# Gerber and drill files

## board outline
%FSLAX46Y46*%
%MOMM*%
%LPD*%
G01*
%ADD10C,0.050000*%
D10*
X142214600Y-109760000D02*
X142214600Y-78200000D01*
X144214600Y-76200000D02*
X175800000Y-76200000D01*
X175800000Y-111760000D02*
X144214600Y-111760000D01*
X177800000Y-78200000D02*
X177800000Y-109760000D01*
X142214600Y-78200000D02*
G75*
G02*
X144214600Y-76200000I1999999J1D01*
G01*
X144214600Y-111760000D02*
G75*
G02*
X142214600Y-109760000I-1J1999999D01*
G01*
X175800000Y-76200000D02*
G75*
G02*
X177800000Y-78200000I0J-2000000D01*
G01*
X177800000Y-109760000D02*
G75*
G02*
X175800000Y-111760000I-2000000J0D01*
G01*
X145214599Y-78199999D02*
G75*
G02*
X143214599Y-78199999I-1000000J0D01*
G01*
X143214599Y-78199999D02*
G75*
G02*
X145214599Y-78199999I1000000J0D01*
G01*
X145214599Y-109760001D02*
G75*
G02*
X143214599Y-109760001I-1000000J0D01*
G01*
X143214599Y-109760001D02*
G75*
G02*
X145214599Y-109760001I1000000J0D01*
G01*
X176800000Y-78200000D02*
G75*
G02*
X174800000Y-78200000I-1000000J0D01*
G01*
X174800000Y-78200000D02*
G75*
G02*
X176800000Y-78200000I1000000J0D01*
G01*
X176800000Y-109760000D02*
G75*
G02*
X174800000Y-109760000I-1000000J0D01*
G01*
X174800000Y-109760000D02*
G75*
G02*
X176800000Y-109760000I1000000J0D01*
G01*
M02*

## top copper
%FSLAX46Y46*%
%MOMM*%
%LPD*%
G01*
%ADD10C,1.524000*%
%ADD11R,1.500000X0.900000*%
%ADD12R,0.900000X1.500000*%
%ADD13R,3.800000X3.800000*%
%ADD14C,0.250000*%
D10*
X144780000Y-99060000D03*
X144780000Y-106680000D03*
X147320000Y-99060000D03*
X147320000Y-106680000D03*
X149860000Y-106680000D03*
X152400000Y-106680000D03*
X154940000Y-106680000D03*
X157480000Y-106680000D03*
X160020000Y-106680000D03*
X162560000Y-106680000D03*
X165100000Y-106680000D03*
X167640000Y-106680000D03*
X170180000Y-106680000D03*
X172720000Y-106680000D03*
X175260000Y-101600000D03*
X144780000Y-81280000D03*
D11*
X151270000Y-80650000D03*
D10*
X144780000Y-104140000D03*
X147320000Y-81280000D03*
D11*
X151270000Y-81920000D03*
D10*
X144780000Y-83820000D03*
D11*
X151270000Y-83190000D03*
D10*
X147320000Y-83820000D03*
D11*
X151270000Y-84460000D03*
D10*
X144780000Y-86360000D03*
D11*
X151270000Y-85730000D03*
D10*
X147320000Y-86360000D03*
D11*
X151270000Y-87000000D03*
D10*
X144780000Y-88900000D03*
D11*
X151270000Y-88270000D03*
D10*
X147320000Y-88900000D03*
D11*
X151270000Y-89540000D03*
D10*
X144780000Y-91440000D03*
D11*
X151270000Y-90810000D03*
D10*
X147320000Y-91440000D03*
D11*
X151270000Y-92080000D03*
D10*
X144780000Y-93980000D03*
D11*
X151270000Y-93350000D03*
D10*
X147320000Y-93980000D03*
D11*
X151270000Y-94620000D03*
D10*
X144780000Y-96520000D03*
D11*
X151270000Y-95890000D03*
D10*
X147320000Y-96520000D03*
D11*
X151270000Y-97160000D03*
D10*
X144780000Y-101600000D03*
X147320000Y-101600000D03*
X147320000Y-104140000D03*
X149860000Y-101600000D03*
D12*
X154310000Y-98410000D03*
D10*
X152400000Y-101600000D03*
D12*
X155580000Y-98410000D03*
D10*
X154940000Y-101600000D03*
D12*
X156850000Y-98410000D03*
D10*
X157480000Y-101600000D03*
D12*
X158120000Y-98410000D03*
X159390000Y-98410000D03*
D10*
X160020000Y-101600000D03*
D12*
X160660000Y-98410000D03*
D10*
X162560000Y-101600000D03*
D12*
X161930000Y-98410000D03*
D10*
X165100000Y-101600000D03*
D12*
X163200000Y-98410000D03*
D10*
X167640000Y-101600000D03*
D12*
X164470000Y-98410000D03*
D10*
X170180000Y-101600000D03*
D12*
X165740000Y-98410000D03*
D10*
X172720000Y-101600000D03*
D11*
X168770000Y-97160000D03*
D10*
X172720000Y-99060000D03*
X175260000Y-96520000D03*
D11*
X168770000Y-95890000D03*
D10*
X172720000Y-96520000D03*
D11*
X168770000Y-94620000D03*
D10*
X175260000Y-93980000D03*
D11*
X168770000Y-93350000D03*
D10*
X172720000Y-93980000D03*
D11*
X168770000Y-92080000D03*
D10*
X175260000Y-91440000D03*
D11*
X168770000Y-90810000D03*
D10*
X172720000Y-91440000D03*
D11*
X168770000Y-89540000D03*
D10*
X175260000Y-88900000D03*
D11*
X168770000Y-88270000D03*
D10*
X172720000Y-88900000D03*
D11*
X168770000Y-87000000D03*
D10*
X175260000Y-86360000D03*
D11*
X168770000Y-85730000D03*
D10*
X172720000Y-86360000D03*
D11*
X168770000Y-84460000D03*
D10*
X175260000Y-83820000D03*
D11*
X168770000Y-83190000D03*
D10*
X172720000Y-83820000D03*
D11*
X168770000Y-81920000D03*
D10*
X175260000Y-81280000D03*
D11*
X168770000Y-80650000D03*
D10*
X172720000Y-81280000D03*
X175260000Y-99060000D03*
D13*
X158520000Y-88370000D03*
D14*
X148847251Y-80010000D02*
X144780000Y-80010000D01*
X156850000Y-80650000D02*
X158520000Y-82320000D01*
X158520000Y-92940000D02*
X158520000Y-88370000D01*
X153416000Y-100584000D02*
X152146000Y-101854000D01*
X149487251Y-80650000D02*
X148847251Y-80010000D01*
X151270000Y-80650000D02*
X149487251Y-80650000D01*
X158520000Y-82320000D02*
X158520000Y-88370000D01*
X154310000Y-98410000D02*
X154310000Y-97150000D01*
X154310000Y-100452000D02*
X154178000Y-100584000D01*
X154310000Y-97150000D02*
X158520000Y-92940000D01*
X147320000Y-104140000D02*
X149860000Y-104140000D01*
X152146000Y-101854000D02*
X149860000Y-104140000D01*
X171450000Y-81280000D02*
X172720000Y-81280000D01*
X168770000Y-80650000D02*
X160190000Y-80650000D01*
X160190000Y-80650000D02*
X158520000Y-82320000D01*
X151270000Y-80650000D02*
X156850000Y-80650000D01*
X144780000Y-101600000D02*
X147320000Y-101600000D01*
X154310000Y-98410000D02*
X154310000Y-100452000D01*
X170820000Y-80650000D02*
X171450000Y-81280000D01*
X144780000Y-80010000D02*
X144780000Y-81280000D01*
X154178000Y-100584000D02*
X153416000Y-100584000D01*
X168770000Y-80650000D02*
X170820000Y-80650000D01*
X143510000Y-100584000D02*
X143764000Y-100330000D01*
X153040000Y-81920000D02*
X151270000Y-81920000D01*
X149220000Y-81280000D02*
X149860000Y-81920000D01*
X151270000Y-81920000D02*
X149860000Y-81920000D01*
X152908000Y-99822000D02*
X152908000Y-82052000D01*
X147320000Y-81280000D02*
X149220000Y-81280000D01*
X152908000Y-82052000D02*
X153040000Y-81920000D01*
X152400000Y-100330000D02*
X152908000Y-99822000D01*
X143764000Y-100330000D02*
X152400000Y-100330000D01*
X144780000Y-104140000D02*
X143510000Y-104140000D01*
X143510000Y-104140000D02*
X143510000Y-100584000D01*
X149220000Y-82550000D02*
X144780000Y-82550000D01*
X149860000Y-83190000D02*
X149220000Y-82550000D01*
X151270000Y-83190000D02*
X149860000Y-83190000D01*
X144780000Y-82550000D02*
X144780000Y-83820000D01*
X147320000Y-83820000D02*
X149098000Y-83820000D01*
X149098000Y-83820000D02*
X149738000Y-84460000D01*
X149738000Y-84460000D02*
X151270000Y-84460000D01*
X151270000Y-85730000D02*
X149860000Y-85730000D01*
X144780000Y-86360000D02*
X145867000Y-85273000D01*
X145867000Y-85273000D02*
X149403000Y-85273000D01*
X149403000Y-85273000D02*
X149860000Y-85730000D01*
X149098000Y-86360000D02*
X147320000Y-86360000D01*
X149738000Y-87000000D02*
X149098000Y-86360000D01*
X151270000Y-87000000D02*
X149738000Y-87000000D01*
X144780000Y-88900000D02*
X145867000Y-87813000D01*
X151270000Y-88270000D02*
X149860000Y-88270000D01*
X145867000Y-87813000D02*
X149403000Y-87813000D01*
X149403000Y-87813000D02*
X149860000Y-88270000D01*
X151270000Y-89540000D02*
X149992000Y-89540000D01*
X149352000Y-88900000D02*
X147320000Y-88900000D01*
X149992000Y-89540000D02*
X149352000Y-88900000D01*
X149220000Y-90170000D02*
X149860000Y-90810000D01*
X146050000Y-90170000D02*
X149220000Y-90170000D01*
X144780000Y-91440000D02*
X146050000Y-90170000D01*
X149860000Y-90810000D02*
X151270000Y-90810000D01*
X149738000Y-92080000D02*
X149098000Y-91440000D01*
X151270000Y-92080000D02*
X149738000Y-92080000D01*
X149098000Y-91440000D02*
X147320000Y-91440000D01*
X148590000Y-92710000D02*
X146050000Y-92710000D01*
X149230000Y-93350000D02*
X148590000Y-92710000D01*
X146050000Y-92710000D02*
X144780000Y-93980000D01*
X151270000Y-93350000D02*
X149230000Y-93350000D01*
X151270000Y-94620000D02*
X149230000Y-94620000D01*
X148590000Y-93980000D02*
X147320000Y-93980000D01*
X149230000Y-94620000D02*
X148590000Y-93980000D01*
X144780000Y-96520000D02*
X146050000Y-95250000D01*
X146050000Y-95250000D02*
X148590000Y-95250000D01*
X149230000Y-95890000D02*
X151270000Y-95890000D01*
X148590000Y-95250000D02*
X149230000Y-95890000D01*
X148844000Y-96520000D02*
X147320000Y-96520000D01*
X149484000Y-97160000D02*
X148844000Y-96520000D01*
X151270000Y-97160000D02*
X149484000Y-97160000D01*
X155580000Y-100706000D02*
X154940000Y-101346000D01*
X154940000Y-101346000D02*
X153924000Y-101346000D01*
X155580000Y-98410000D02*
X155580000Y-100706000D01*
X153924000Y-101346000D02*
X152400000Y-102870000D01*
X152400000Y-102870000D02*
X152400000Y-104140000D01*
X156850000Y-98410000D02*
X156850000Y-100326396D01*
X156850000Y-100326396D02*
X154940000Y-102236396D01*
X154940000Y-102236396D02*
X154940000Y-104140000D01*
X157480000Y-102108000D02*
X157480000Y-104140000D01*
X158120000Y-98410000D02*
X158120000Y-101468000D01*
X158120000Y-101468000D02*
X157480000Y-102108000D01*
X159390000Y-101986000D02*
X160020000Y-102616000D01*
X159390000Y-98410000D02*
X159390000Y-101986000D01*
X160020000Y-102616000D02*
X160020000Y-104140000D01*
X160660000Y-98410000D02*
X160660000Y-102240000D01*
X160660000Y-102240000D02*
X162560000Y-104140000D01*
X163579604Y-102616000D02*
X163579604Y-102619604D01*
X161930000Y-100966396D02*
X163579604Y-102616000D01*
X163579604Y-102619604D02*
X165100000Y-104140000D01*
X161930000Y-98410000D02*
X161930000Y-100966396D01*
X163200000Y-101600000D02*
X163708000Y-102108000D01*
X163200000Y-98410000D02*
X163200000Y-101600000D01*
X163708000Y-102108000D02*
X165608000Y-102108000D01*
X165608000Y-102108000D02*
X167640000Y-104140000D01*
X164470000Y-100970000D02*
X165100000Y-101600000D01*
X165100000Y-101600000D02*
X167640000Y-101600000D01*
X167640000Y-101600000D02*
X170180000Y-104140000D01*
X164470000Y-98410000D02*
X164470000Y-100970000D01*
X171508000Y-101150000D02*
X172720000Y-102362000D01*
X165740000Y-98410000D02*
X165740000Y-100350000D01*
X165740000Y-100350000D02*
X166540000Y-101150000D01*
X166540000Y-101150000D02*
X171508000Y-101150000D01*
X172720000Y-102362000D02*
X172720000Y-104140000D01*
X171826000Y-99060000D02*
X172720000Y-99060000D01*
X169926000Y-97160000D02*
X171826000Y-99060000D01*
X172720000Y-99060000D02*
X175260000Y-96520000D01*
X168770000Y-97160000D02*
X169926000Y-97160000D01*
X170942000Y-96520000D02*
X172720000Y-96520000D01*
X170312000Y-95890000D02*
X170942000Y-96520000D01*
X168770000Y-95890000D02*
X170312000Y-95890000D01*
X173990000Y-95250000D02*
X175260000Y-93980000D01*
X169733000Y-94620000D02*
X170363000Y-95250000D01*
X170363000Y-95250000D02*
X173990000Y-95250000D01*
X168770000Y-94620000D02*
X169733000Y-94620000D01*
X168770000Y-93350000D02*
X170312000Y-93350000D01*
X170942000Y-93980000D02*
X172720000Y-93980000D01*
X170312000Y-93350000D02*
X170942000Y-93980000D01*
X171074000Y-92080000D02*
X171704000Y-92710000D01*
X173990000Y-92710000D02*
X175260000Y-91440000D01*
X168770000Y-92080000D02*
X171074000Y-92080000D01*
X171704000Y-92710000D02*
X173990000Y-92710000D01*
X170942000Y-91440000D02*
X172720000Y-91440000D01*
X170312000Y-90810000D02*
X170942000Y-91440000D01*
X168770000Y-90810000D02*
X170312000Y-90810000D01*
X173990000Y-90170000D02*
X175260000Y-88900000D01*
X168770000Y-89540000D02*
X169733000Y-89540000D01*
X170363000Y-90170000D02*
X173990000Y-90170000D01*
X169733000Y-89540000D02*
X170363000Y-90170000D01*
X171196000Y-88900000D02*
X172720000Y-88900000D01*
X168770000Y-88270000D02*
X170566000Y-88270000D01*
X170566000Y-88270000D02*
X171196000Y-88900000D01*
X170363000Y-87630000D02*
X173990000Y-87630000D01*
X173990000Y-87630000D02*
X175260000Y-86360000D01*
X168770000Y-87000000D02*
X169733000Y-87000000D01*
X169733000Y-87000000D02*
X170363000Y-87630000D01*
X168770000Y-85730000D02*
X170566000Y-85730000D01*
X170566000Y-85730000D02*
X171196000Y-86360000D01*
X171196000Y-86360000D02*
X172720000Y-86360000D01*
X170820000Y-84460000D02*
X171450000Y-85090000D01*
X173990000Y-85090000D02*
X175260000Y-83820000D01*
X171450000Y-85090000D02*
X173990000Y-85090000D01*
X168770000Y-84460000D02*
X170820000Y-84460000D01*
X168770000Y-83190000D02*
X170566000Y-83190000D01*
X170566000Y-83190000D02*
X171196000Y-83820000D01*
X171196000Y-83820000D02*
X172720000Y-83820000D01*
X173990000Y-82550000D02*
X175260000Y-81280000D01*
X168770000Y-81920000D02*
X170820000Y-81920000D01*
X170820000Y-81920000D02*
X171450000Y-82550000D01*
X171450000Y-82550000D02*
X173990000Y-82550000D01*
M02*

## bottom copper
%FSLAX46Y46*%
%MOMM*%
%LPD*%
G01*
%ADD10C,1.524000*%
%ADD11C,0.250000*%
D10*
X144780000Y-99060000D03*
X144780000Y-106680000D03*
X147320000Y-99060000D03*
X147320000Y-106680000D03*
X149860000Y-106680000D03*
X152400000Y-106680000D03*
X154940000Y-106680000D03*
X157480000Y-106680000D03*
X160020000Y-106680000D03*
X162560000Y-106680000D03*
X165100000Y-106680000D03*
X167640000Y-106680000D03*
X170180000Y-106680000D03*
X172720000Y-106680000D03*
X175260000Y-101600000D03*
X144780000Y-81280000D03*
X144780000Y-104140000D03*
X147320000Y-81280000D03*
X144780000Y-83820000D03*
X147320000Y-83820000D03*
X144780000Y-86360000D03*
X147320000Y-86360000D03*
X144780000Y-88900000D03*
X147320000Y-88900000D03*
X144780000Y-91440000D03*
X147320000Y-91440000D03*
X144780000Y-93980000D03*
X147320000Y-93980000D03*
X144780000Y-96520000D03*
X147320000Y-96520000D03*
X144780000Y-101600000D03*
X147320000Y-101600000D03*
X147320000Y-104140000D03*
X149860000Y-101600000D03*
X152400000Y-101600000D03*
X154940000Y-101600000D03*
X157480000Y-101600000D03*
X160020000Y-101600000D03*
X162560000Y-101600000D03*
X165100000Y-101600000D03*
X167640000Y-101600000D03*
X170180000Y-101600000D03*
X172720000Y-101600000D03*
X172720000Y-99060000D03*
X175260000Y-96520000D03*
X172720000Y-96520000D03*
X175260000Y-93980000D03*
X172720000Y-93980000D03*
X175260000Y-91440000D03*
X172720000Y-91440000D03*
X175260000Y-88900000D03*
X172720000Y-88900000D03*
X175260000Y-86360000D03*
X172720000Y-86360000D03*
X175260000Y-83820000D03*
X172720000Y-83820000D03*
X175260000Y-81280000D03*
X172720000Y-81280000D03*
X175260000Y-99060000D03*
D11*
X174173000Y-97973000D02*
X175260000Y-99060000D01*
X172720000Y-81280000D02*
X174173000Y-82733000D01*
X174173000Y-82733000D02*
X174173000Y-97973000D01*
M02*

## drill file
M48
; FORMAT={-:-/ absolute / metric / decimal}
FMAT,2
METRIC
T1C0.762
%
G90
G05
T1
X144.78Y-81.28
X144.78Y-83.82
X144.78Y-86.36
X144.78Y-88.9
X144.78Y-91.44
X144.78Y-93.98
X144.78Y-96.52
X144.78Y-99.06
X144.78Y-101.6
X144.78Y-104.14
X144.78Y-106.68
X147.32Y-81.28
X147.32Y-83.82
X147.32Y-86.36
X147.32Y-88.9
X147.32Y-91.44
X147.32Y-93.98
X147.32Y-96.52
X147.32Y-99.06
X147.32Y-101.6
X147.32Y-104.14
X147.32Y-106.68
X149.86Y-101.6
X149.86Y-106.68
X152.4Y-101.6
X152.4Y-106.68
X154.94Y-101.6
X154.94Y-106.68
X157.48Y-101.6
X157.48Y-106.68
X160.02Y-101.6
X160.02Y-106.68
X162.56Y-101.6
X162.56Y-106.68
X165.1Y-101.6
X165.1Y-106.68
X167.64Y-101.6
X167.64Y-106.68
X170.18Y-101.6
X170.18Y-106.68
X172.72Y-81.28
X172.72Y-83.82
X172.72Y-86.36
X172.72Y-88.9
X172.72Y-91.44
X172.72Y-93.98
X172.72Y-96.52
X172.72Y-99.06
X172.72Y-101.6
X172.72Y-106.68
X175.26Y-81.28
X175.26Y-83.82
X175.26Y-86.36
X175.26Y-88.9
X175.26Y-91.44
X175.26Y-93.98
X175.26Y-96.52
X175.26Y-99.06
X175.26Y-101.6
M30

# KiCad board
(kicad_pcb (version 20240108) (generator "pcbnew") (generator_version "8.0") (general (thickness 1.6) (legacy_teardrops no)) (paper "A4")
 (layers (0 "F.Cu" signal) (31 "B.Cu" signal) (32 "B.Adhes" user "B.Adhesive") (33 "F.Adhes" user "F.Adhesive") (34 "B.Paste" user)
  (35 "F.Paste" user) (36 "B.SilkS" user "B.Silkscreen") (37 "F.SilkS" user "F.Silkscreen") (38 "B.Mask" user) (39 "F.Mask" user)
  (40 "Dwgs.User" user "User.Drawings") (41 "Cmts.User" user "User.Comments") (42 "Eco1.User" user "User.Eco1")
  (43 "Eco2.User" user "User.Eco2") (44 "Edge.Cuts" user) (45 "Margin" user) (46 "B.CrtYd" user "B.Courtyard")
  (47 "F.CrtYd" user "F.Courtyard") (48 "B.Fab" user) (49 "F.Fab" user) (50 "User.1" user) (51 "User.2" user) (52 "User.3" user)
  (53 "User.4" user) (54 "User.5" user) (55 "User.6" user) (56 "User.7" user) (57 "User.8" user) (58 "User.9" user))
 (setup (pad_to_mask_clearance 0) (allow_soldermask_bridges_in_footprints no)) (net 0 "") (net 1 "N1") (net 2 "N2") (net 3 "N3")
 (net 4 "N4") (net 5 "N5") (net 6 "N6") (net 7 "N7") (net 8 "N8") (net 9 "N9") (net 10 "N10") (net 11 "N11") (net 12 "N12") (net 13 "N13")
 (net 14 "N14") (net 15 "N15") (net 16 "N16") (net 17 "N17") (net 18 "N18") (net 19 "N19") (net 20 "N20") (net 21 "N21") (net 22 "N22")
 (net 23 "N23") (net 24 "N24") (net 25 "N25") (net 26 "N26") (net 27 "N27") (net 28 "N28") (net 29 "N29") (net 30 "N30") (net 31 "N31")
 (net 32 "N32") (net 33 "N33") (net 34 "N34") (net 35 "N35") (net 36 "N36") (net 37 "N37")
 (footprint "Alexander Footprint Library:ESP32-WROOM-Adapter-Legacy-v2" (layer "F.Cu") (at 160.02 88.9)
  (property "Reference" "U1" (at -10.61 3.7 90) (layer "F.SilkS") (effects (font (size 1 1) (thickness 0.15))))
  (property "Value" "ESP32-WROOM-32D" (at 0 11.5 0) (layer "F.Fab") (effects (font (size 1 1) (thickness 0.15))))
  (fp_line (start -17.8054 20.86) (end -17.8054 -10.7) (stroke (width 0.05) (type default)) (layer "Edge.Cuts"))
  (fp_line (start -15.8054 -12.7) (end 15.78 -12.7) (stroke (width 0.05) (type default)) (layer "Edge.Cuts"))
  (fp_line (start 15.78 22.86) (end -15.8054 22.86) (stroke (width 0.05) (type default)) (layer "Edge.Cuts"))
  (fp_line (start 17.78 -10.7) (end 17.78 20.86) (stroke (width 0.05) (type default)) (layer "Edge.Cuts"))
  (fp_arc (start -17.8054 -10.7) (mid -17.219614 -12.114214) (end -15.8054 -12.7) (stroke (width 0.05) (type default)) (layer "Edge.Cuts"))
  (fp_arc (start -15.8054 22.86) (mid -17.219614 22.274214) (end -17.8054 20.86) (stroke (width 0.05) (type default)) (layer "Edge.Cuts"))
  (fp_arc (start 15.78 -12.7) (mid 17.194214 -12.114214) (end 17.78 -10.7) (stroke (width 0.05) (type default)) (layer "Edge.Cuts"))
  (fp_arc (start 17.78 20.86) (mid 17.194214 22.274214) (end 15.78 22.86) (stroke (width 0.05) (type default)) (layer "Edge.Cuts"))
  (fp_circle (center -15.805401 -10.700001) (end -14.805401 -10.700001) (stroke (width 0.05) (type default)) (fill none) (layer "Edge.Cuts"))
  (fp_circle (center -15.805401 20.860001) (end -14.805401 20.860001) (stroke (width 0.05) (type default)) (fill none) (layer "Edge.Cuts"))
  (fp_circle (center 15.78 -10.7) (end 16.78 -10.7) (stroke (width 0.05) (type default)) (fill none) (layer "Edge.Cuts"))
  (fp_circle (center 15.78 20.86) (end 16.78 20.86) (stroke (width 0.05) (type default)) (fill none) (layer "Edge.Cuts"))
  (pad "" thru_hole circle (at -15.24 10.16) (size 1.524 1.524) (drill 0.762) (layers "*.Cu" "*.Mask") (remove_unused_layers no))
  (pad "" thru_hole circle (at -15.24 17.78 90) (size 1.524 1.524) (drill 0.762) (layers "*.Cu" "*.Mask") (remove_unused_layers no))
  (pad "" thru_hole circle (at -12.7 10.16) (size 1.524 1.524) (drill 0.762) (layers "*.Cu" "*.Mask") (remove_unused_layers no))
  (pad "" thru_hole circle (at -12.7 17.78 90) (size 1.524 1.524) (drill 0.762) (layers "*.Cu" "*.Mask") (remove_unused_layers no))
  (pad "" thru_hole circle (at -10.16 17.78 90) (size 1.524 1.524) (drill 0.762) (layers "*.Cu" "*.Mask") (remove_unused_layers no))
  (pad "" thru_hole circle (at -7.62 17.78 90) (size 1.524 1.524) (drill 0.762) (layers "*.Cu" "*.Mask") (remove_unused_layers no))
  (pad "" thru_hole circle (at -5.08 17.78 90) (size 1.524 1.524) (drill 0.762) (layers "*.Cu" "*.Mask") (remove_unused_layers no))
  (pad "" thru_hole circle (at -2.54 17.78 90) (size 1.524 1.524) (drill 0.762) (layers "*.Cu" "*.Mask") (remove_unused_layers no))
  (pad "" thru_hole circle (at 0 17.78 90) (size 1.524 1.524) (drill 0.762) (layers "*.Cu" "*.Mask") (remove_unused_layers no))
  (pad "" thru_hole circle (at 2.54 17.78 90) (size 1.524 1.524) (drill 0.762) (layers "*.Cu" "*.Mask") (remove_unused_layers no))
  (pad "" thru_hole circle (at 5.08 17.78 90) (size 1.524 1.524) (drill 0.762) (layers "*.Cu" "*.Mask") (remove_unused_layers no))
  (pad "" thru_hole circle (at 7.62 17.78 90) (size 1.524 1.524) (drill 0.762) (layers "*.Cu" "*.Mask") (remove_unused_layers no))
  (pad "" thru_hole circle (at 10.16 17.78 90) (size 1.524 1.524) (drill 0.762) (layers "*.Cu" "*.Mask") (remove_unused_layers no))
  (pad "" thru_hole circle (at 12.7 17.78 90) (size 1.524 1.524) (drill 0.762) (layers "*.Cu" "*.Mask") (remove_unused_layers no))
  (pad "" thru_hole circle (at 15.24 12.7 90) (size 1.524 1.524) (drill 0.762) (layers "*.Cu" "*.Mask") (remove_unused_layers no))
  (pad "1" thru_hole circle (at -15.24 -7.62) (size 1.524 1.524) (drill 0.762) (layers "*.Cu" "*.Mask") (remove_unused_layers no)
   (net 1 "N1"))
  (pad "1" smd rect (at -8.75 -8.25) (size 1.5 0.9) (layers "F.Cu" "F.Paste" "F.Mask") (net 1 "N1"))
  (pad "2" thru_hole circle (at -15.24 15.24 90) (size 1.524 1.524) (drill 0.762) (layers "*.Cu" "*.Mask") (remove_unused_layers no)
   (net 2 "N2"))
  (pad "2" thru_hole circle (at -12.7 -7.62) (size 1.524 1.524) (drill 0.762) (layers "*.Cu" "*.Mask") (remove_unused_layers no)
   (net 2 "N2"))
  (pad "2" smd rect (at -8.75 -6.98) (size 1.5 0.9) (layers "F.Cu" "F.Paste" "F.Mask") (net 2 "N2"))
  (pad "3" thru_hole circle (at -15.24 -5.08) (size 1.524 1.524) (drill 0.762) (layers "*.Cu" "*.Mask") (remove_unused_layers no)
   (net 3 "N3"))
  (pad "3" smd rect (at -8.75 -5.71) (size 1.5 0.9) (layers "F.Cu" "F.Paste" "F.Mask") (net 3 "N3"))
  (pad "4" thru_hole circle (at -12.7 -5.08) (size 1.524 1.524) (drill 0.762) (layers "*.Cu" "*.Mask") (remove_unused_layers no)
   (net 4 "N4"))
  (pad "4" smd rect (at -8.75 -4.44) (size 1.5 0.9) (layers "F.Cu" "F.Paste" "F.Mask") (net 4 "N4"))
  (pad "5" thru_hole circle (at -15.24 -2.54) (size 1.524 1.524) (drill 0.762) (layers "*.Cu" "*.Mask") (remove_unused_layers no)
   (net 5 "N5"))
  (pad "5" smd rect (at -8.75 -3.17) (size 1.5 0.9) (layers "F.Cu" "F.Paste" "F.Mask") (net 5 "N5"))
  (pad "6" thru_hole circle (at -12.7 -2.54) (size 1.524 1.524) (drill 0.762) (layers "*.Cu" "*.Mask") (remove_unused_layers no)
   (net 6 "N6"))
  (pad "6" smd rect (at -8.75 -1.9) (size 1.5 0.9) (layers "F.Cu" "F.Paste" "F.Mask") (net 6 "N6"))
  (pad "7" thru_hole circle (at -15.24 0) (size 1.524 1.524) (drill 0.762) (layers "*.Cu" "*.Mask") (remove_unused_layers no) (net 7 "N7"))
  (pad "7" smd rect (at -8.75 -0.63) (size 1.5 0.9) (layers "F.Cu" "F.Paste" "F.Mask") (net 7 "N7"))
  (pad "8" thru_hole circle (at -12.7 0) (size 1.524 1.524) (drill 0.762) (layers "*.Cu" "*.Mask") (remove_unused_layers no) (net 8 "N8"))
  (pad "8" smd rect (at -8.75 0.64) (size 1.5 0.9) (layers "F.Cu" "F.Paste" "F.Mask") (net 8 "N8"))
  (pad "9" thru_hole circle (at -15.24 2.54) (size 1.524 1.524) (drill 0.762) (layers "*.Cu" "*.Mask") (remove_unused_layers no)
   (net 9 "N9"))
  (pad "9" smd rect (at -8.75 1.91) (size 1.5 0.9) (layers "F.Cu" "F.Paste" "F.Mask") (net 9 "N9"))
  (pad "10" thru_hole circle (at -12.7 2.54) (size 1.524 1.524) (drill 0.762) (layers "*.Cu" "*.Mask") (remove_unused_layers no)
   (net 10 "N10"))
  (pad "10" smd rect (at -8.75 3.18) (size 1.5 0.9) (layers "F.Cu" "F.Paste" "F.Mask") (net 10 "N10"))
  (pad "11" thru_hole circle (at -15.24 5.08) (size 1.524 1.524) (drill 0.762) (layers "*.Cu" "*.Mask") (remove_unused_layers no)
   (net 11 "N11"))
  (pad "11" smd rect (at -8.75 4.45) (size 1.5 0.9) (layers "F.Cu" "F.Paste" "F.Mask") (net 11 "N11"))
  (pad "12" thru_hole circle (at -12.7 5.08) (size 1.524 1.524) (drill 0.762) (layers "*.Cu" "*.Mask") (remove_unused_layers no)
   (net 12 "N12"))
  (pad "12" smd rect (at -8.75 5.72) (size 1.5 0.9) (layers "F.Cu" "F.Paste" "F.Mask") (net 12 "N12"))
  (pad "13" thru_hole circle (at -15.24 7.62) (size 1.524 1.524) (drill 0.762) (layers "*.Cu" "*.Mask") (remove_unused_layers no)
   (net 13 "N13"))
  (pad "13" smd rect (at -8.75 6.99) (size 1.5 0.9) (layers "F.Cu" "F.Paste" "F.Mask") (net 13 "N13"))
  (pad "14" thru_hole circle (at -12.7 7.62) (size 1.524 1.524) (drill 0.762) (layers "*.Cu" "*.Mask") (remove_unused_layers no)
   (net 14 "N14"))
  (pad "14" smd rect (at -8.75 8.26) (size 1.5 0.9) (layers "F.Cu" "F.Paste" "F.Mask") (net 14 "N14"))
  (pad "15" thru_hole circle (at -15.24 12.7 90) (size 1.524 1.524) (drill 0.762) (layers "*.Cu" "*.Mask") (remove_unused_layers no)
   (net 1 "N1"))
  (pad "15" thru_hole circle (at -12.7 12.7 90) (size 1.524 1.524) (drill 0.762) (layers "*.Cu" "*.Mask") (remove_unused_layers no)
   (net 1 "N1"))
  (pad "15" thru_hole circle (at -12.7 15.24 90) (size 1.524 1.524) (drill 0.762) (layers "*.Cu" "*.Mask") (remove_unused_layers no)
   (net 1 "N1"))
  (pad "15" thru_hole circle (at -10.16 12.7 90) (size 1.524 1.524) (drill 0.762) (layers "*.Cu" "*.Mask") (remove_unused_layers no)
   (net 1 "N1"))
  (pad "15" smd rect (at -5.71 9.51 90) (size 1.5 0.9) (layers "F.Cu" "F.Paste" "F.Mask") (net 1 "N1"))
  (pad "16" thru_hole circle (at -7.62 12.7 90) (size 1.524 1.524) (drill 0.762) (layers "*.Cu" "*.Mask") (remove_unused_layers no)
   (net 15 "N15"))
  (pad "16" smd rect (at -4.44 9.51 90) (size 1.5 0.9) (layers "F.Cu" "F.Paste" "F.Mask") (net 15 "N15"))
  (pad "17" thru_hole circle (at -5.08 12.7 90) (size 1.524 1.524) (drill 0.762) (layers "*.Cu" "*.Mask") (remove_unused_layers no)
   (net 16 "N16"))
  (pad "17" smd rect (at -3.17 9.51 90) (size 1.5 0.9) (layers "F.Cu" "F.Paste" "F.Mask") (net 16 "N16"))
  (pad "18" thru_hole circle (at -2.54 12.7 90) (size 1.524 1.524) (drill 0.762) (layers "*.Cu" "*.Mask") (remove_unused_layers no)
   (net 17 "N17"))
  (pad "18" smd rect (at -1.9 9.51 90) (size 1.5 0.9) (layers "F.Cu" "F.Paste" "F.Mask") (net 17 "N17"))
  (pad "19" smd rect (at -0.63 9.51 90) (size 1.5 0.9) (layers "F.Cu" "F.Paste" "F.Mask") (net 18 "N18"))
  (pad "19" thru_hole circle (at 0 12.7 90) (size 1.524 1.524) (drill 0.762) (layers "*.Cu" "*.Mask") (remove_unused_layers no)
   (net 18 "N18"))
  (pad "20" smd rect (at 0.64 9.51 90) (size 1.5 0.9) (layers "F.Cu" "F.Paste" "F.Mask") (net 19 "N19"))
  (pad "20" thru_hole circle (at 2.54 12.7 90) (size 1.524 1.524) (drill 0.762) (layers "*.Cu" "*.Mask") (remove_unused_layers no)
   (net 19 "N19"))
  (pad "21" smd rect (at 1.91 9.51 90) (size 1.5 0.9) (layers "F.Cu" "F.Paste" "F.Mask") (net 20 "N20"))
  (pad "21" thru_hole circle (at 5.08 12.7 90) (size 1.524 1.524) (drill 0.762) (layers "*.Cu" "*.Mask") (remove_unused_layers no)
   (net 20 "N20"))
  (pad "22" smd rect (at 3.18 9.51 90) (size 1.5 0.9) (layers "F.Cu" "F.Paste" "F.Mask") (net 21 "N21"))
  (pad "22" thru_hole circle (at 7.62 12.7 90) (size 1.524 1.524) (drill 0.762) (layers "*.Cu" "*.Mask") (remove_unused_layers no)
   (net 21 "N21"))
  (pad "23" smd rect (at 4.45 9.51 90) (size 1.5 0.9) (layers "F.Cu" "F.Paste" "F.Mask") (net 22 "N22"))
  (pad "23" thru_hole circle (at 10.16 12.7 90) (size 1.524 1.524) (drill 0.762) (layers "*.Cu" "*.Mask") (remove_unused_layers no)
   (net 22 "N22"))
  (pad "24" smd rect (at 5.72 9.51 90) (size 1.5 0.9) (layers "F.Cu" "F.Paste" "F.Mask") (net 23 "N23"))
  (pad "24" thru_hole circle (at 12.7 12.7 90) (size 1.524 1.524) (drill 0.762) (layers "*.Cu" "*.Mask") (remove_unused_layers no)
   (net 23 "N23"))
  (pad "25" smd rect (at 8.75 8.26) (size 1.5 0.9) (layers "F.Cu" "F.Paste" "F.Mask") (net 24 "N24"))
  (pad "25" thru_hole circle (at 12.7 10.16) (size 1.524 1.524) (drill 0.762) (layers "*.Cu" "*.Mask") (remove_unused_layers no)
   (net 24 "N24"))
  (pad "25" thru_hole circle (at 15.24 7.62) (size 1.524 1.524) (drill 0.762) (layers "*.Cu" "*.Mask") (remove_unused_layers no)
   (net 24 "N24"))
  (pad "26" smd rect (at 8.75 6.99) (size 1.5 0.9) (layers "F.Cu" "F.Paste" "F.Mask") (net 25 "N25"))
  (pad "26" thru_hole circle (at 12.7 7.62) (size 1.524 1.524) (drill 0.762) (layers "*.Cu" "*.Mask") (remove_unused_layers no)
   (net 25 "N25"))
  (pad "27" smd rect (at 8.75 5.72) (size 1.5 0.9) (layers "F.Cu" "F.Paste" "F.Mask") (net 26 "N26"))
  (pad "27" thru_hole circle (at 15.24 5.08) (size 1.524 1.524) (drill 0.762) (layers "*.Cu" "*.Mask") (remove_unused_layers no)
   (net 26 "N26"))
  (pad "28" smd rect (at 8.75 4.45) (size 1.5 0.9) (layers "F.Cu" "F.Paste" "F.Mask") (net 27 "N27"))
  (pad "28" thru_hole circle (at 12.7 5.08) (size 1.524 1.524) (drill 0.762) (layers "*.Cu" "*.Mask") (remove_unused_layers no)
   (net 27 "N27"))
  (pad "29" smd rect (at 8.75 3.18) (size 1.5 0.9) (layers "F.Cu" "F.Paste" "F.Mask") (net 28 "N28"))
  (pad "29" thru_hole circle (at 15.24 2.54) (size 1.524 1.524) (drill 0.762) (layers "*.Cu" "*.Mask") (remove_unused_layers no)
   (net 28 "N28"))
  (pad "30" smd rect (at 8.75 1.91) (size 1.5 0.9) (layers "F.Cu" "F.Paste" "F.Mask") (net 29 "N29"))
  (pad "30" thru_hole circle (at 12.7 2.54) (size 1.524 1.524) (drill 0.762) (layers "*.Cu" "*.Mask") (remove_unused_layers no)
   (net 29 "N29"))
  (pad "31" smd rect (at 8.75 0.64) (size 1.5 0.9) (layers "F.Cu" "F.Paste" "F.Mask") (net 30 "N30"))
  (pad "31" thru_hole circle (at 15.24 0) (size 1.524 1.524) (drill 0.762) (layers "*.Cu" "*.Mask") (remove_unused_layers no) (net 30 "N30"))
  (pad "32" smd rect (at 8.75 -0.63) (size 1.5 0.9) (layers "F.Cu" "F.Paste" "F.Mask") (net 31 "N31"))
  (pad "32" thru_hole circle (at 12.7 0) (size 1.524 1.524) (drill 0.762) (layers "*.Cu" "*.Mask") (remove_unused_layers no) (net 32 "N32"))
  (pad "33" smd rect (at 8.75 -1.9) (size 1.5 0.9) (layers "F.Cu" "F.Paste" "F.Mask") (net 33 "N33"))
  (pad "33" thru_hole circle (at 15.24 -2.54) (size 1.524 1.524) (drill 0.762) (layers "*.Cu" "*.Mask") (remove_unused_layers no)
   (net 33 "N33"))
  (pad "34" smd rect (at 8.75 -3.17) (size 1.5 0.9) (layers "F.Cu" "F.Paste" "F.Mask") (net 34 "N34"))
  (pad "34" thru_hole circle (at 12.7 -2.54) (size 1.524 1.524) (drill 0.762) (layers "*.Cu" "*.Mask") (remove_unused_layers no)
   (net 34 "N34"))
  (pad "35" smd rect (at 8.75 -4.44) (size 1.5 0.9) (layers "F.Cu" "F.Paste" "F.Mask") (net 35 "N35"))
  (pad "35" thru_hole circle (at 15.24 -5.08) (size 1.524 1.524) (drill 0.762) (layers "*.Cu" "*.Mask") (remove_unused_layers no)
   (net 35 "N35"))
  (pad "36" smd rect (at 8.75 -5.71) (size 1.5 0.9) (layers "F.Cu" "F.Paste" "F.Mask") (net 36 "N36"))
  (pad "36" thru_hole circle (at 12.7 -5.08) (size 1.524 1.524) (drill 0.762) (layers "*.Cu" "*.Mask") (remove_unused_layers no)
   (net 36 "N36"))
  (pad "37" smd rect (at 8.75 -6.98) (size 1.5 0.9) (layers "F.Cu" "F.Paste" "F.Mask") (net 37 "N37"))
  (pad "37" thru_hole circle (at 15.24 -7.62) (size 1.524 1.524) (drill 0.762) (layers "*.Cu" "*.Mask") (remove_unused_layers no)
   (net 37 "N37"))
  (pad "38" smd rect (at 8.75 -8.25) (size 1.5 0.9) (layers "F.Cu" "F.Paste" "F.Mask") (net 1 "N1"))
  (pad "38" thru_hole circle (at 12.7 -7.62) (size 1.524 1.524) (drill 0.762) (layers "*.Cu" "*.Mask") (remove_unused_layers no)
   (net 1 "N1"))
  (pad "38" thru_hole circle (at 15.24 10.16) (size 1.524 1.524) (drill 0.762) (layers "*.Cu" "*.Mask") (remove_unused_layers no)
   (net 1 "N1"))
  (pad "39" smd rect (at -1.5 -0.53) (size 3.8 3.8) (layers "F.Cu" "F.Mask") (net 1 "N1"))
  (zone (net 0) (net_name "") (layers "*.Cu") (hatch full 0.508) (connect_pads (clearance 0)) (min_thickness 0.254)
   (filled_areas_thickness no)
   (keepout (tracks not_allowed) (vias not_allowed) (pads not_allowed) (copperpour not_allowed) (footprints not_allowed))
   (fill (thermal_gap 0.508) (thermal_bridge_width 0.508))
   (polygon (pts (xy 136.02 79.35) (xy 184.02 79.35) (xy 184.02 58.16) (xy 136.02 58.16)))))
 (segment (start 148.847251 80.01) (end 144.78 80.01) (width 0.25) (layer "F.Cu") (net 1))
 (segment (start 156.85 80.65) (end 158.52 82.32) (width 0.25) (layer "F.Cu") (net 1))
 (segment (start 158.52 92.94) (end 158.52 88.37) (width 0.25) (layer "F.Cu") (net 1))
 (segment (start 153.416 100.584) (end 152.146 101.854) (width 0.25) (layer "F.Cu") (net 1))
 (segment (start 149.487251 80.65) (end 148.847251 80.01) (width 0.25) (layer "F.Cu") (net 1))
 (segment (start 151.27 80.65) (end 149.487251 80.65) (width 0.25) (layer "F.Cu") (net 1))
 (segment (start 158.52 82.32) (end 158.52 88.37) (width 0.25) (layer "F.Cu") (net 1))
 (segment (start 154.31 98.41) (end 154.31 97.15) (width 0.25) (layer "F.Cu") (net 1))
 (segment (start 154.31 100.452) (end 154.178 100.584) (width 0.25) (layer "F.Cu") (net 1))
 (segment (start 154.31 97.15) (end 158.52 92.94) (width 0.25) (layer "F.Cu") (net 1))
 (segment (start 147.32 104.14) (end 149.86 104.14) (width 0.25) (layer "F.Cu") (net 1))
 (segment (start 152.146 101.854) (end 149.86 104.14) (width 0.25) (layer "F.Cu") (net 1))
 (segment (start 171.45 81.28) (end 172.72 81.28) (width 0.25) (layer "F.Cu") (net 1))
 (segment (start 168.77 80.65) (end 160.19 80.65) (width 0.25) (layer "F.Cu") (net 1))
 (segment (start 160.19 80.65) (end 158.52 82.32) (width 0.25) (layer "F.Cu") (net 1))
 (segment (start 151.27 80.65) (end 156.85 80.65) (width 0.25) (layer "F.Cu") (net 1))
 (segment (start 144.78 101.6) (end 147.32 101.6) (width 0.25) (layer "F.Cu") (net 1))
 (segment (start 154.31 98.41) (end 154.31 100.452) (width 0.25) (layer "F.Cu") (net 1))
 (segment (start 170.82 80.65) (end 171.45 81.28) (width 0.25) (layer "F.Cu") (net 1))
 (segment (start 144.78 80.01) (end 144.78 81.28) (width 0.25) (layer "F.Cu") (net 1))
 (segment (start 154.178 100.584) (end 153.416 100.584) (width 0.25) (layer "F.Cu") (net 1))
 (segment (start 168.77 80.65) (end 170.82 80.65) (width 0.25) (layer "F.Cu") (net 1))
 (segment (start 174.173 97.973) (end 175.26 99.06) (width 0.25) (layer "B.Cu") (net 1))
 (segment (start 172.72 81.28) (end 174.173 82.733) (width 0.25) (layer "B.Cu") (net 1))
 (segment (start 174.173 82.733) (end 174.173 97.973) (width 0.25) (layer "B.Cu") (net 1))
 (segment (start 143.51 100.584) (end 143.764 100.33) (width 0.25) (layer "F.Cu") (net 2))
 (segment (start 153.04 81.92) (end 151.27 81.92) (width 0.25) (layer "F.Cu") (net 2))
 (segment (start 149.22 81.28) (end 149.86 81.92) (width 0.25) (layer "F.Cu") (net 2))
 (segment (start 151.27 81.92) (end 149.86 81.92) (width 0.25) (layer "F.Cu") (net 2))
 (segment (start 152.908 99.822) (end 152.908 82.052) (width 0.25) (layer "F.Cu") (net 2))
 (segment (start 147.32 81.28) (end 149.22 81.28) (width 0.25) (layer "F.Cu") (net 2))
 (segment (start 152.908 82.052) (end 153.04 81.92) (width 0.25) (layer "F.Cu") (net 2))
 (segment (start 152.4 100.33) (end 152.908 99.822) (width 0.25) (layer "F.Cu") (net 2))
 (segment (start 143.764 100.33) (end 152.4 100.33) (width 0.25) (layer "F.Cu") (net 2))
 (segment (start 144.78 104.14) (end 143.51 104.14) (width 0.25) (layer "F.Cu") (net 2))
 (segment (start 143.51 104.14) (end 143.51 100.584) (width 0.25) (layer "F.Cu") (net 2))
 (segment (start 149.22 82.55) (end 144.78 82.55) (width 0.25) (layer "F.Cu") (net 3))
 (segment (start 149.86 83.19) (end 149.22 82.55) (width 0.25) (layer "F.Cu") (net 3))
 (segment (start 151.27 83.19) (end 149.86 83.19) (width 0.25) (layer "F.Cu") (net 3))
 (segment (start 144.78 82.55) (end 144.78 83.82) (width 0.25) (layer "F.Cu") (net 3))
 (segment (start 147.32 83.82) (end 149.098 83.82) (width 0.25) (layer "F.Cu") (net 4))
 (segment (start 149.098 83.82) (end 149.738 84.46) (width 0.25) (layer "F.Cu") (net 4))
 (segment (start 149.738 84.46) (end 151.27 84.46) (width 0.25) (layer "F.Cu") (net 4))
 (segment (start 151.27 85.73) (end 149.86 85.73) (width 0.25) (layer "F.Cu") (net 5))
 (segment (start 144.78 86.36) (end 145.867 85.273) (width 0.25) (layer "F.Cu") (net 5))
 (segment (start 145.867 85.273) (end 149.403 85.273) (width 0.25) (layer "F.Cu") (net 5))
 (segment (start 149.403 85.273) (end 149.86 85.73) (width 0.25) (layer "F.Cu") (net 5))
 (segment (start 149.098 86.36) (end 147.32 86.36) (width 0.25) (layer "F.Cu") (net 6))
 (segment (start 149.738 87) (end 149.098 86.36) (width 0.25) (layer "F.Cu") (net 6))
 (segment (start 151.27 87) (end 149.738 87) (width 0.25) (layer "F.Cu") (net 6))
 (segment (start 144.78 88.9) (end 145.867 87.813) (width 0.25) (layer "F.Cu") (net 7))
 (segment (start 151.27 88.27) (end 149.86 88.27) (width 0.25) (layer "F.Cu") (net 7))
 (segment (start 145.867 87.813) (end 149.403 87.813) (width 0.25) (layer "F.Cu") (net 7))
 (segment (start 149.403 87.813) (end 149.86 88.27) (width 0.25) (layer "F.Cu") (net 7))
 (segment (start 151.27 89.54) (end 149.992 89.54) (width 0.25) (layer "F.Cu") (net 8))
 (segment (start 149.352 88.9) (end 147.32 88.9) (width 0.25) (layer "F.Cu") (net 8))
 (segment (start 149.992 89.54) (end 149.352 88.9) (width 0.25) (layer "F.Cu") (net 8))
 (segment (start 149.22 90.17) (end 149.86 90.81) (width 0.25) (layer "F.Cu") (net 9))
 (segment (start 146.05 90.17) (end 149.22 90.17) (width 0.25) (layer "F.Cu") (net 9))
 (segment (start 144.78 91.44) (end 146.05 90.17) (width 0.25) (layer "F.Cu") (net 9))
 (segment (start 149.86 90.81) (end 151.27 90.81) (width 0.25) (layer "F.Cu") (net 9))
 (segment (start 149.738 92.08) (end 149.098 91.44) (width 0.25) (layer "F.Cu") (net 10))
 (segment (start 151.27 92.08) (end 149.738 92.08) (width 0.25) (layer "F.Cu") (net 10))
 (segment (start 149.098 91.44) (end 147.32 91.44) (width 0.25) (layer "F.Cu") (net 10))
 (segment (start 148.59 92.71) (end 146.05 92.71) (width 0.25) (layer "F.Cu") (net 11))
 (segment (start 149.23 93.35) (end 148.59 92.71) (width 0.25) (layer "F.Cu") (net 11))
 (segment (start 146.05 92.71) (end 144.78 93.98) (width 0.25) (layer "F.Cu") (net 11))
 (segment (start 151.27 93.35) (end 149.23 93.35) (width 0.25) (layer "F.Cu") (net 11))
 (segment (start 151.27 94.62) (end 149.23 94.62) (width 0.25) (layer "F.Cu") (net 12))
 (segment (start 148.59 93.98) (end 147.32 93.98) (width 0.25) (layer "F.Cu") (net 12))
 (segment (start 149.23 94.62) (end 148.59 93.98) (width 0.25) (layer "F.Cu") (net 12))
 (segment (start 144.78 96.52) (end 146.05 95.25) (width 0.25) (layer "F.Cu") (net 13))
 (segment (start 146.05 95.25) (end 148.59 95.25) (width 0.25) (layer "F.Cu") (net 13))
 (segment (start 149.23 95.89) (end 151.27 95.89) (width 0.25) (layer "F.Cu") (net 13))
 (segment (start 148.59 95.25) (end 149.23 95.89) (width 0.25) (layer "F.Cu") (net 13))
 (segment (start 148.844 96.52) (end 147.32 96.52) (width 0.25) (layer "F.Cu") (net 14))
 (segment (start 149.484 97.16) (end 148.844 96.52) (width 0.25) (layer "F.Cu") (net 14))
 (segment (start 151.27 97.16) (end 149.484 97.16) (width 0.25) (layer "F.Cu") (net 14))
 (segment (start 155.58 100.706) (end 154.94 101.346) (width 0.25) (layer "F.Cu") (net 15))
 (segment (start 154.94 101.346) (end 153.924 101.346) (width 0.25) (layer "F.Cu") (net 15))
 (segment (start 155.58 98.41) (end 155.58 100.706) (width 0.25) (layer "F.Cu") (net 15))
 (segment (start 153.924 101.346) (end 152.4 102.87) (width 0.25) (layer "F.Cu") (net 15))
 (segment (start 152.4 102.87) (end 152.4 104.14) (width 0.25) (layer "F.Cu") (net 15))
 (segment (start 156.85 98.41) (end 156.85 100.326396) (width 0.25) (layer "F.Cu") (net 16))
 (segment (start 156.85 100.326396) (end 154.94 102.236396) (width 0.25) (layer "F.Cu") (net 16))
 (segment (start 154.94 102.236396) (end 154.94 104.14) (width 0.25) (layer "F.Cu") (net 16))
 (segment (start 157.48 102.108) (end 157.48 104.14) (width 0.25) (layer "F.Cu") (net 17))
 (segment (start 158.12 98.41) (end 158.12 101.468) (width 0.25) (layer "F.Cu") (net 17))
 (segment (start 158.12 101.468) (end 157.48 102.108) (width 0.25) (layer "F.Cu") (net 17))
 (segment (start 159.39 101.986) (end 160.02 102.616) (width 0.25) (layer "F.Cu") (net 18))
 (segment (start 159.39 98.41) (end 159.39 101.986) (width 0.25) (layer "F.Cu") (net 18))
 (segment (start 160.02 102.616) (end 160.02 104.14) (width 0.25) (layer "F.Cu") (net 18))
 (segment (start 160.66 98.41) (end 160.66 102.24) (width 0.25) (layer "F.Cu") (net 19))
 (segment (start 160.66 102.24) (end 162.56 104.14) (width 0.25) (layer "F.Cu") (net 19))
 (segment (start 163.579604 102.616) (end 163.579604 102.619604) (width 0.25) (layer "F.Cu") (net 20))
 (segment (start 161.93 100.966396) (end 163.579604 102.616) (width 0.25) (layer "F.Cu") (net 20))
 (segment (start 163.579604 102.619604) (end 165.1 104.14) (width 0.25) (layer "F.Cu") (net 20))
 (segment (start 161.93 98.41) (end 161.93 100.966396) (width 0.25) (layer "F.Cu") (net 20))
 (segment (start 163.2 101.6) (end 163.708 102.108) (width 0.25) (layer "F.Cu") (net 21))
 (segment (start 163.2 98.41) (end 163.2 101.6) (width 0.25) (layer "F.Cu") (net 21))
 (segment (start 163.708 102.108) (end 165.608 102.108) (width 0.25) (layer "F.Cu") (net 21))
 (segment (start 165.608 102.108) (end 167.64 104.14) (width 0.25) (layer "F.Cu") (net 21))
 (segment (start 164.47 100.97) (end 165.1 101.6) (width 0.25) (layer "F.Cu") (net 22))
 (segment (start 165.1 101.6) (end 167.64 101.6) (width 0.25) (layer "F.Cu") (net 22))
 (segment (start 167.64 101.6) (end 170.18 104.14) (width 0.25) (layer "F.Cu") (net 22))
 (segment (start 164.47 98.41) (end 164.47 100.97) (width 0.25) (layer "F.Cu") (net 22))
 (segment (start 171.508 101.15) (end 172.72 102.362) (width 0.25) (layer "F.Cu") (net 23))
 (segment (start 165.74 98.41) (end 165.74 100.35) (width 0.25) (layer "F.Cu") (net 23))
 (segment (start 165.74 100.35) (end 166.54 101.15) (width 0.25) (layer "F.Cu") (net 23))
 (segment (start 166.54 101.15) (end 171.508 101.15) (width 0.25) (layer "F.Cu") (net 23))
 (segment (start 172.72 102.362) (end 172.72 104.14) (width 0.25) (layer "F.Cu") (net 23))
 (segment (start 171.826 99.06) (end 172.72 99.06) (width 0.25) (layer "F.Cu") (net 24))
 (segment (start 169.926 97.16) (end 171.826 99.06) (width 0.25) (layer "F.Cu") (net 24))
 (segment (start 172.72 99.06) (end 175.26 96.52) (width 0.25) (layer "F.Cu") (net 24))
 (segment (start 168.77 97.16) (end 169.926 97.16) (width 0.25) (layer "F.Cu") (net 24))
 (segment (start 170.942 96.52) (end 172.72 96.52) (width 0.25) (layer "F.Cu") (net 25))
 (segment (start 170.312 95.89) (end 170.942 96.52) (width 0.25) (layer "F.Cu") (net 25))
 (segment (start 168.77 95.89) (end 170.312 95.89) (width 0.25) (layer "F.Cu") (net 25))
 (segment (start 173.99 95.25) (end 175.26 93.98) (width 0.25) (layer "F.Cu") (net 26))
 (segment (start 169.733 94.62) (end 170.363 95.25) (width 0.25) (layer "F.Cu") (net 26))
 (segment (start 170.363 95.25) (end 173.99 95.25) (width 0.25) (layer "F.Cu") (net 26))
 (segment (start 168.77 94.62) (end 169.733 94.62) (width 0.25) (layer "F.Cu") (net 26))
 (segment (start 168.77 93.35) (end 170.312 93.35) (width 0.25) (layer "F.Cu") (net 27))
 (segment (start 170.942 93.98) (end 172.72 93.98) (width 0.25) (layer "F.Cu") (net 27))
 (segment (start 170.312 93.35) (end 170.942 93.98) (width 0.25) (layer "F.Cu") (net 27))
 (segment (start 171.074 92.08) (end 171.704 92.71) (width 0.25) (layer "F.Cu") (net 28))
 (segment (start 173.99 92.71) (end 175.26 91.44) (width 0.25) (layer "F.Cu") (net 28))
 (segment (start 168.77 92.08) (end 171.074 92.08) (width 0.25) (layer "F.Cu") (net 28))
 (segment (start 171.704 92.71) (end 173.99 92.71) (width 0.25) (layer "F.Cu") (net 28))
 (segment (start 170.942 91.44) (end 172.72 91.44) (width 0.25) (layer "F.Cu") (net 29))
 (segment (start 170.312 90.81) (end 170.942 91.44) (width 0.25) (layer "F.Cu") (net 29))
 (segment (start 168.77 90.81) (end 170.312 90.81) (width 0.25) (layer "F.Cu") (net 29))
 (segment (start 173.99 90.17) (end 175.26 88.9) (width 0.25) (layer "F.Cu") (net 30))
 (segment (start 168.77 89.54) (end 169.733 89.54) (width 0.25) (layer "F.Cu") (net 30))
 (segment (start 170.363 90.17) (end 173.99 90.17) (width 0.25) (layer "F.Cu") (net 30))
 (segment (start 169.733 89.54) (end 170.363 90.17) (width 0.25) (layer "F.Cu") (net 30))
 (segment (start 171.196 88.9) (end 172.72 88.9) (width 0.25) (layer "F.Cu") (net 32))
 (segment (start 168.77 88.27) (end 170.566 88.27) (width 0.25) (layer "F.Cu") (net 32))
 (segment (start 170.566 88.27) (end 171.196 88.9) (width 0.25) (layer "F.Cu") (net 32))
 (segment (start 170.363 87.63) (end 173.99 87.63) (width 0.25) (layer "F.Cu") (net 33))
 (segment (start 173.99 87.63) (end 175.26 86.36) (width 0.25) (layer "F.Cu") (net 33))
 (segment (start 168.77 87) (end 169.733 87) (width 0.25) (layer "F.Cu") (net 33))
 (segment (start 169.733 87) (end 170.363 87.63) (width 0.25) (layer "F.Cu") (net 33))
 (segment (start 168.77 85.73) (end 170.566 85.73) (width 0.25) (layer "F.Cu") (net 34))
 (segment (start 170.566 85.73) (end 171.196 86.36) (width 0.25) (layer "F.Cu") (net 34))
 (segment (start 171.196 86.36) (end 172.72 86.36) (width 0.25) (layer "F.Cu") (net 34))
 (segment (start 170.82 84.46) (end 171.45 85.09) (width 0.25) (layer "F.Cu") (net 35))
 (segment (start 173.99 85.09) (end 175.26 83.82) (width 0.25) (layer "F.Cu") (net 35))
 (segment (start 171.45 85.09) (end 173.99 85.09) (width 0.25) (layer "F.Cu") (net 35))
 (segment (start 168.77 84.46) (end 170.82 84.46) (width 0.25) (layer "F.Cu") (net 35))
 (segment (start 168.77 83.19) (end 170.566 83.19) (width 0.25) (layer "F.Cu") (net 36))
 (segment (start 170.566 83.19) (end 171.196 83.82) (width 0.25) (layer "F.Cu") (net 36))
 (segment (start 171.196 83.82) (end 172.72 83.82) (width 0.25) (layer "F.Cu") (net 36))
 (segment (start 173.99 82.55) (end 175.26 81.28) (width 0.25) (layer "F.Cu") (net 37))
 (segment (start 168.77 81.92) (end 170.82 81.92) (width 0.25) (layer "F.Cu") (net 37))
 (segment (start 170.82 81.92) (end 171.45 82.55) (width 0.25) (layer "F.Cu") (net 37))
 (segment (start 171.45 82.55) (end 173.99 82.55) (width 0.25) (layer "F.Cu") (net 37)))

